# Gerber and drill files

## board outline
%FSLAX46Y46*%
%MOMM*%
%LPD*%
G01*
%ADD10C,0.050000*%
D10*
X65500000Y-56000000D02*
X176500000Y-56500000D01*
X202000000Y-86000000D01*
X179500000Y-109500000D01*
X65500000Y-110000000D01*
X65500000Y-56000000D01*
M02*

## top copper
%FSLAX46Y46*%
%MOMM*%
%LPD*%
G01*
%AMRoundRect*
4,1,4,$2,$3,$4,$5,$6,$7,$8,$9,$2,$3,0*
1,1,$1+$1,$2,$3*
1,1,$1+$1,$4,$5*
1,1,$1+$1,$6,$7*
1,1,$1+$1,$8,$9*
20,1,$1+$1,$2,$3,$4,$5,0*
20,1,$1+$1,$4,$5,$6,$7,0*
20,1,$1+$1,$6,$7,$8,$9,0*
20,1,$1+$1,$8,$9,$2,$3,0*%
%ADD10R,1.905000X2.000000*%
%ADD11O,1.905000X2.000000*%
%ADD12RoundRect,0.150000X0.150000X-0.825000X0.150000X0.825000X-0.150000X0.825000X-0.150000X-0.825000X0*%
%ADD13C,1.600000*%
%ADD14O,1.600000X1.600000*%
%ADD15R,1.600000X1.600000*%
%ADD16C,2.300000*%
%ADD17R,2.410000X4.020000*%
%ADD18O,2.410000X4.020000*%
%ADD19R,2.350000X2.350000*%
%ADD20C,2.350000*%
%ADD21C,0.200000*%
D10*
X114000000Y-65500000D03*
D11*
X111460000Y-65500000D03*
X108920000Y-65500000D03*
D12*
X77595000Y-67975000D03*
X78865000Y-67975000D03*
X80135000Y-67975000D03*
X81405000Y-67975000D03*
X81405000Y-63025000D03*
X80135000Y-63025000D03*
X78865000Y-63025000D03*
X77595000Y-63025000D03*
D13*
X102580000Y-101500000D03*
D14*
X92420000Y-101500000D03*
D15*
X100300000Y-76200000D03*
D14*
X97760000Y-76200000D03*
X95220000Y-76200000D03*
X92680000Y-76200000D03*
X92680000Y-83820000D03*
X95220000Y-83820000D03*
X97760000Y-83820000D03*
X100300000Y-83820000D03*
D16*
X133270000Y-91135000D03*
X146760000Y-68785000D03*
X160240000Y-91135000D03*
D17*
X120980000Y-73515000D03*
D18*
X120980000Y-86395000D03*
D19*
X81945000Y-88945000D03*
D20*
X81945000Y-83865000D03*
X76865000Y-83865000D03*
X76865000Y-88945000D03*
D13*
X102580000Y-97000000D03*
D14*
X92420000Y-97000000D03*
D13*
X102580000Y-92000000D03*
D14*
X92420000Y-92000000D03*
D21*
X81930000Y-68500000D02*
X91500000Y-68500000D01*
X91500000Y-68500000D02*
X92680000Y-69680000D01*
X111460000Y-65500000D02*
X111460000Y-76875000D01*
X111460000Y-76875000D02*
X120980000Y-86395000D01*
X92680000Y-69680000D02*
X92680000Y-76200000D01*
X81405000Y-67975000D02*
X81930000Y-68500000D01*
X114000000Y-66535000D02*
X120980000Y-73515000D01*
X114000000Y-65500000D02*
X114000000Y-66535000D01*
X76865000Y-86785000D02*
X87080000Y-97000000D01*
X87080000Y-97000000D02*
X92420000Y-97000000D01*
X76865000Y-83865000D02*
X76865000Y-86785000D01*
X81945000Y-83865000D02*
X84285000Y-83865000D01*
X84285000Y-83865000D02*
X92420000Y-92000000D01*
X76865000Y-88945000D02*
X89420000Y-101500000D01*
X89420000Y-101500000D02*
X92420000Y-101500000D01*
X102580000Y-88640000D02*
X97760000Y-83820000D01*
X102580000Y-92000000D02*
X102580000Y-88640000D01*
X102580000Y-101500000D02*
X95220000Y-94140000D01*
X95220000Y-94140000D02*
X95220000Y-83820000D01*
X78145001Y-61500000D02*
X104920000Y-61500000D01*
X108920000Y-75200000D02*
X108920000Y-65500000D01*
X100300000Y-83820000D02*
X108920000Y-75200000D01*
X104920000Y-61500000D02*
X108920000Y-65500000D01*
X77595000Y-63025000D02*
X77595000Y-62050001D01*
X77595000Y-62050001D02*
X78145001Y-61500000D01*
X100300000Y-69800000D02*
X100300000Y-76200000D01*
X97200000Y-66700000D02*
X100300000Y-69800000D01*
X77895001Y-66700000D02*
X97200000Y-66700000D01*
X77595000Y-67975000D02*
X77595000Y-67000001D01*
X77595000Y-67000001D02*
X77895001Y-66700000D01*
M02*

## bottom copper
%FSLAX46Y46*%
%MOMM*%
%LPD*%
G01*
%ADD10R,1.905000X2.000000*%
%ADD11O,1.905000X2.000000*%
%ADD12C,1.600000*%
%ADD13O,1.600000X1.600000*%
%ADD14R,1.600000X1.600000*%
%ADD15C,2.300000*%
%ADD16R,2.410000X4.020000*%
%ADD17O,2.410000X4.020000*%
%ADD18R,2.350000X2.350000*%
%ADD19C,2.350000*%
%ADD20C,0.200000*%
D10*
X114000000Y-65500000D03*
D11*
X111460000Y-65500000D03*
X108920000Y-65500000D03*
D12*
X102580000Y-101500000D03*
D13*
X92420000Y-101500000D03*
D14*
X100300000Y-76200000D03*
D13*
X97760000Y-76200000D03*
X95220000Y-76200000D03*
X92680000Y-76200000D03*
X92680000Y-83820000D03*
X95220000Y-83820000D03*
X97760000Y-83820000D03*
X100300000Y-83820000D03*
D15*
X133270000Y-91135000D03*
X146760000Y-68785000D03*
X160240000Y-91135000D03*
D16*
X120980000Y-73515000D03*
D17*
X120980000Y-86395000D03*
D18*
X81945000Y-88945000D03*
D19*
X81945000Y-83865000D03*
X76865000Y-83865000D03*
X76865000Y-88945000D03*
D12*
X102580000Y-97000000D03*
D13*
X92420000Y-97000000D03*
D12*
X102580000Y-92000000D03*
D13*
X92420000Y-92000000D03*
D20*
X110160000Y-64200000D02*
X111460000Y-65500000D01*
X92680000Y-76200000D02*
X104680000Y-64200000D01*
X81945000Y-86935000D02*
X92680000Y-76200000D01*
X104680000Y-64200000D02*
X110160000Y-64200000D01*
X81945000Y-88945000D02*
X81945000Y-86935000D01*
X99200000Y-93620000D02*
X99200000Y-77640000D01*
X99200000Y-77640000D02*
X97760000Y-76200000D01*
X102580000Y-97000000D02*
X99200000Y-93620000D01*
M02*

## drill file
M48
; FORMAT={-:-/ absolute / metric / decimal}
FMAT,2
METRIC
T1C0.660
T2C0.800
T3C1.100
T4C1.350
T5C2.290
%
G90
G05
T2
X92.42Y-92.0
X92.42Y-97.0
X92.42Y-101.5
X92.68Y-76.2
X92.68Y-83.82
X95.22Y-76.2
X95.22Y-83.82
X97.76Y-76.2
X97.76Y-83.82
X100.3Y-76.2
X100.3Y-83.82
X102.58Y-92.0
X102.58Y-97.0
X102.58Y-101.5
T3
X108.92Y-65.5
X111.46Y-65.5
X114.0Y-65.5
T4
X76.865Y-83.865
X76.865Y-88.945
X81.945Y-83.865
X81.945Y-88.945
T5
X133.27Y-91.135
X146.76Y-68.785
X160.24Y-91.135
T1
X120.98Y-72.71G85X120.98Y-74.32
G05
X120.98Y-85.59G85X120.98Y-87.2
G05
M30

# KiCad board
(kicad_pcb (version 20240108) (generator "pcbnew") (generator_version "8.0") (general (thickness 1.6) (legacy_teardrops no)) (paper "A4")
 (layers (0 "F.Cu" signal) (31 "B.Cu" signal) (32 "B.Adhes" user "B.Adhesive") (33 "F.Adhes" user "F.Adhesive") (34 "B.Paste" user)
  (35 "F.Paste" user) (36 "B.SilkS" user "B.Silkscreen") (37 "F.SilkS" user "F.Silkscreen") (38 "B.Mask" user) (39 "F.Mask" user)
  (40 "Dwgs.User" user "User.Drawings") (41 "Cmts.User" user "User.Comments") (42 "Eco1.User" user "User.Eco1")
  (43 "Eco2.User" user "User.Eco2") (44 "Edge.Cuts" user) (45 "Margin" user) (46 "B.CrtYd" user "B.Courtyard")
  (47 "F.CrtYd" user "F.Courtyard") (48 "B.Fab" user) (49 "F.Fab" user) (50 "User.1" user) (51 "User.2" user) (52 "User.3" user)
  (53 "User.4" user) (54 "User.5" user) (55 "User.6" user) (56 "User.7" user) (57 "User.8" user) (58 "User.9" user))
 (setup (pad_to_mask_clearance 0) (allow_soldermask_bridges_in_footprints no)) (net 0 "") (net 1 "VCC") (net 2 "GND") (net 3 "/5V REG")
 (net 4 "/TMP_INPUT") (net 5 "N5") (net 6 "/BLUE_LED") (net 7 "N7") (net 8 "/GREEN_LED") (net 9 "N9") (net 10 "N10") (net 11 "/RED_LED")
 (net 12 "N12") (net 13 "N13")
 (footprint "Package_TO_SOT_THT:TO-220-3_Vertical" (layer "F.Cu") (at 114 65.5 180)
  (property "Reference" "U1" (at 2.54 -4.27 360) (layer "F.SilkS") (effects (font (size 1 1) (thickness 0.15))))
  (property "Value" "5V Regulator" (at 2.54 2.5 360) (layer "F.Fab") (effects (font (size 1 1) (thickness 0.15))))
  (pad "1" thru_hole rect (at 0 0 180) (size 1.905 2) (drill 1.1) (layers "*.Cu" "*.Mask") (remove_unused_layers no) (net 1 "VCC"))
  (pad "2" thru_hole oval (at 2.54 0 180) (size 1.905 2) (drill 1.1) (layers "*.Cu" "*.Mask") (remove_unused_layers no) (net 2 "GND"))
  (pad "3" thru_hole oval (at 5.08 0 180) (size 1.905 2) (drill 1.1) (layers "*.Cu" "*.Mask") (remove_unused_layers no) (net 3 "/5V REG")))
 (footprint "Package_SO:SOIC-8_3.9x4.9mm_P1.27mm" (layer "F.Cu") (at 79.5 65.5 90)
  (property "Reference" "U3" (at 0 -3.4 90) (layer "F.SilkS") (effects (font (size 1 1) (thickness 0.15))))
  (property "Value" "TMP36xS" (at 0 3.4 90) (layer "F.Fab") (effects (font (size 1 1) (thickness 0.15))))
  (pad "1" smd roundrect (at -2.475 -1.905 90) (size 1.95 0.6) (layers "F.Cu" "F.Paste" "F.Mask") (roundrect_rratio 0.25)
   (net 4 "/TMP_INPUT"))
  (pad "2" smd roundrect (at -2.475 -0.635 90) (size 1.95 0.6) (layers "F.Cu" "F.Paste" "F.Mask") (roundrect_rratio 0.25))
  (pad "3" smd roundrect (at -2.475 0.635 90) (size 1.95 0.6) (layers "F.Cu" "F.Paste" "F.Mask") (roundrect_rratio 0.25))
  (pad "4" smd roundrect (at -2.475 1.905 90) (size 1.95 0.6) (layers "F.Cu" "F.Paste" "F.Mask") (roundrect_rratio 0.25) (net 2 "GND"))
  (pad "5" smd roundrect (at 2.475 1.905 90) (size 1.95 0.6) (layers "F.Cu" "F.Paste" "F.Mask") (roundrect_rratio 0.25) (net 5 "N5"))
  (pad "6" smd roundrect (at 2.475 0.635 90) (size 1.95 0.6) (layers "F.Cu" "F.Paste" "F.Mask") (roundrect_rratio 0.25))
  (pad "7" smd roundrect (at 2.475 -0.635 90) (size 1.95 0.6) (layers "F.Cu" "F.Paste" "F.Mask") (roundrect_rratio 0.25))
  (pad "8" smd roundrect (at 2.475 -1.905 90) (size 1.95 0.6) (layers "F.Cu" "F.Paste" "F.Mask") (roundrect_rratio 0.25) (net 3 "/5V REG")))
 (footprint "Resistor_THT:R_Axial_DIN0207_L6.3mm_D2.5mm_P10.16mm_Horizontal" (layer "F.Cu") (at 102.58 101.5 180)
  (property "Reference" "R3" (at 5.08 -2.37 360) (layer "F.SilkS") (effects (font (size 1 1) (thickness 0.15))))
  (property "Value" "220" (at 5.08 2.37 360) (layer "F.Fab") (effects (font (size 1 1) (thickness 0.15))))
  (pad "1" thru_hole circle (at 0 0 180) (size 1.6 1.6) (drill 0.8) (layers "*.Cu" "*.Mask") (remove_unused_layers no) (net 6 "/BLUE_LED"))
  (pad "2" thru_hole oval (at 10.16 0 180) (size 1.6 1.6) (drill 0.8) (layers "*.Cu" "*.Mask") (remove_unused_layers no) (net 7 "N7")))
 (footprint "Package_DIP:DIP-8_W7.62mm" (layer "F.Cu") (at 100.3 76.2 -90)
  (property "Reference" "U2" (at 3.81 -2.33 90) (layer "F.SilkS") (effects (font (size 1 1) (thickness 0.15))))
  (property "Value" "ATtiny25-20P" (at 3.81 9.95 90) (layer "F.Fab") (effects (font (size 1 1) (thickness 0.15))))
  (pad "1" thru_hole rect (at 0 0 270) (size 1.6 1.6) (drill 0.8) (layers "*.Cu" "*.Mask") (remove_unused_layers no) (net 4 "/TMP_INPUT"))
  (pad "2" thru_hole oval (at 0 2.54 270) (size 1.6 1.6) (drill 0.8) (layers "*.Cu" "*.Mask") (remove_unused_layers no) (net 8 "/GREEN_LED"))
  (pad "3" thru_hole oval (at 0 5.08 270) (size 1.6 1.6) (drill 0.8) (layers "*.Cu" "*.Mask") (remove_unused_layers no) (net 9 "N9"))
  (pad "4" thru_hole oval (at 0 7.62 270) (size 1.6 1.6) (drill 0.8) (layers "*.Cu" "*.Mask") (remove_unused_layers no) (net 2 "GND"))
  (pad "5" thru_hole oval (at 7.62 7.62 270) (size 1.6 1.6) (drill 0.8) (layers "*.Cu" "*.Mask") (remove_unused_layers no) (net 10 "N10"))
  (pad "6" thru_hole oval (at 7.62 5.08 270) (size 1.6 1.6) (drill 0.8) (layers "*.Cu" "*.Mask") (remove_unused_layers no)
   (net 6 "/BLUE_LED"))
  (pad "7" thru_hole oval (at 7.62 2.54 270) (size 1.6 1.6) (drill 0.8) (layers "*.Cu" "*.Mask") (remove_unused_layers no)
   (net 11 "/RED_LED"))
  (pad "8" thru_hole oval (at 7.62 0 270) (size 1.6 1.6) (drill 0.8) (layers "*.Cu" "*.Mask") (remove_unused_layers no) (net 3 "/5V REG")))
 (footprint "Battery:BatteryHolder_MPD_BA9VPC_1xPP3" (layer "F.Cu") (at 120.98 73.515)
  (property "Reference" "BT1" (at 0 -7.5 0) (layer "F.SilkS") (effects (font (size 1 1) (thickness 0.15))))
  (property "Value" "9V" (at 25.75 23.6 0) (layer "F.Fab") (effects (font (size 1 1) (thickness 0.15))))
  (pad "" np_thru_hole circle (at 12.29 17.62) (size 2.3 2.3) (drill 2.29) (layers "*.Cu" "*.Mask"))
  (pad "" np_thru_hole circle (at 25.78 -4.73) (size 2.3 2.3) (drill 2.29) (layers "*.Cu" "*.Mask"))
  (pad "" np_thru_hole circle (at 39.26 17.62) (size 2.3 2.3) (drill 2.29) (layers "*.Cu" "*.Mask"))
  (pad "1" thru_hole rect (at 0 0) (size 2.41 4.02) (drill oval 0.66 2.27) (layers "*.Cu" "*.Mask") (remove_unused_layers no) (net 1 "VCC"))
  (pad "2" thru_hole oval (at 0 12.88) (size 2.41 4.02) (drill oval 0.66 2.27) (layers "*.Cu" "*.Mask") (remove_unused_layers no)
   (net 2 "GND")))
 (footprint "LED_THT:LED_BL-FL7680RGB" (layer "F.Cu") (at 81.945 88.945 180)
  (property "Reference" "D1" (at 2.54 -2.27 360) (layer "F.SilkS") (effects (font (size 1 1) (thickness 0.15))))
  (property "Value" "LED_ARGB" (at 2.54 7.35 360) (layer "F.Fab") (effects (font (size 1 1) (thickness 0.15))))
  (pad "1" thru_hole rect (at 0 0 180) (size 2.35 2.35) (drill 1.35) (layers "*.Cu" "*.Mask") (remove_unused_layers no) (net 2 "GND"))
  (pad "2" thru_hole circle (at 0 5.08 180) (size 2.35 2.35) (drill 1.35) (layers "*.Cu" "*.Mask") (remove_unused_layers no) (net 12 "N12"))
  (pad "3" thru_hole circle (at 5.08 5.08 180) (size 2.35 2.35) (drill 1.35) (layers "*.Cu" "*.Mask") (remove_unused_layers no)
   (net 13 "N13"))
  (pad "4" thru_hole circle (at 5.08 0 180) (size 2.35 2.35) (drill 1.35) (layers "*.Cu" "*.Mask") (remove_unused_layers no) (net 7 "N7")))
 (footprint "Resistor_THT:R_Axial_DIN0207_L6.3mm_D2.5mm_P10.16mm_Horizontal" (layer "F.Cu") (at 102.58 97 180)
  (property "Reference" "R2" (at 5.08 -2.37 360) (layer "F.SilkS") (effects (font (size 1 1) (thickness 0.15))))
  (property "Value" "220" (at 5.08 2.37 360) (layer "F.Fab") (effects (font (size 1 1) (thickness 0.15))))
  (pad "1" thru_hole circle (at 0 0 180) (size 1.6 1.6) (drill 0.8) (layers "*.Cu" "*.Mask") (remove_unused_layers no) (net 8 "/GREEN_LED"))
  (pad "2" thru_hole oval (at 10.16 0 180) (size 1.6 1.6) (drill 0.8) (layers "*.Cu" "*.Mask") (remove_unused_layers no) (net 13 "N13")))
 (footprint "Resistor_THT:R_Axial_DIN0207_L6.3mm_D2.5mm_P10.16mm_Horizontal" (layer "F.Cu") (at 102.58 92 180)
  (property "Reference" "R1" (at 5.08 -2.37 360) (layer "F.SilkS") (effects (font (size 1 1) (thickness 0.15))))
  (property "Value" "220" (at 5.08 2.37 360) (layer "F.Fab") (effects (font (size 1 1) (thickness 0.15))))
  (pad "1" thru_hole circle (at 0 0 180) (size 1.6 1.6) (drill 0.8) (layers "*.Cu" "*.Mask") (remove_unused_layers no) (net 11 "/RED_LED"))
  (pad "2" thru_hole oval (at 10.16 0 180) (size 1.6 1.6) (drill 0.8) (layers "*.Cu" "*.Mask") (remove_unused_layers no) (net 12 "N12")))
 (gr_poly
  (pts (xy 65.5 56) (xy 176.5 56.5) (xy 202 86) (xy 179.5 109.5) (xy 65.5 110)) (stroke (width 0.05) (type solid)) (fill none)
  (layer "Edge.Cuts"))
 (segment (start 81.93 68.5) (end 91.5 68.5) (width 0.2) (layer "F.Cu") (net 2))
 (segment (start 91.5 68.5) (end 92.68 69.68) (width 0.2) (layer "F.Cu") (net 2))
 (segment (start 111.46 65.5) (end 111.46 76.875) (width 0.2) (layer "F.Cu") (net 2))
 (segment (start 111.46 76.875) (end 120.98 86.395) (width 0.2) (layer "F.Cu") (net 2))
 (segment (start 92.68 69.68) (end 92.68 76.2) (width 0.2) (layer "F.Cu") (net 2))
 (segment (start 81.405 67.975) (end 81.93 68.5) (width 0.2) (layer "F.Cu") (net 2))
 (segment (start 110.16 64.2) (end 111.46 65.5) (width 0.2) (layer "B.Cu") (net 2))
 (segment (start 92.68 76.2) (end 104.68 64.2) (width 0.2) (layer "B.Cu") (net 2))
 (segment (start 81.945 86.935) (end 92.68 76.2) (width 0.2) (layer "B.Cu") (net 2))
 (segment (start 104.68 64.2) (end 110.16 64.2) (width 0.2) (layer "B.Cu") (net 2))
 (segment (start 81.945 88.945) (end 81.945 86.935) (width 0.2) (layer "B.Cu") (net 2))
 (segment (start 114 66.535) (end 120.98 73.515) (width 0.2) (layer "F.Cu") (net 1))
 (segment (start 114 65.5) (end 114 66.535) (width 0.2) (layer "F.Cu") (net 1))
 (segment (start 76.865 86.785) (end 87.08 97) (width 0.2) (layer "F.Cu") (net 13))
 (segment (start 87.08 97) (end 92.42 97) (width 0.2) (layer "F.Cu") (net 13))
 (segment (start 76.865 83.865) (end 76.865 86.785) (width 0.2) (layer "F.Cu") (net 13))
 (segment (start 81.945 83.865) (end 84.285 83.865) (width 0.2) (layer "F.Cu") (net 12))
 (segment (start 84.285 83.865) (end 92.42 92) (width 0.2) (layer "F.Cu") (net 12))
 (segment (start 76.865 88.945) (end 89.42 101.5) (width 0.2) (layer "F.Cu") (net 7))
 (segment (start 89.42 101.5) (end 92.42 101.5) (width 0.2) (layer "F.Cu") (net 7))
 (segment (start 102.58 88.64) (end 97.76 83.82) (width 0.2) (layer "F.Cu") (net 11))
 (segment (start 102.58 92) (end 102.58 88.64) (width 0.2) (layer "F.Cu") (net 11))
 (segment (start 99.2 93.62) (end 99.2 77.64) (width 0.2) (layer "B.Cu") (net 8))
 (segment (start 99.2 77.64) (end 97.76 76.2) (width 0.2) (layer "B.Cu") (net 8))
 (segment (start 102.58 97) (end 99.2 93.62) (width 0.2) (layer "B.Cu") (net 8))
 (segment (start 102.58 101.5) (end 95.22 94.14) (width 0.2) (layer "F.Cu") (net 6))
 (segment (start 95.22 94.14) (end 95.22 83.82) (width 0.2) (layer "F.Cu") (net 6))
 (segment (start 78.145001 61.5) (end 104.92 61.5) (width 0.2) (layer "F.Cu") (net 3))
 (segment (start 108.92 75.2) (end 108.92 65.5) (width 0.2) (layer "F.Cu") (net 3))
 (segment (start 100.3 83.82) (end 108.92 75.2) (width 0.2) (layer "F.Cu") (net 3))
 (segment (start 104.92 61.5) (end 108.92 65.5) (width 0.2) (layer "F.Cu") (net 3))
 (segment (start 77.595 63.025) (end 77.595 62.050001) (width 0.2) (layer "F.Cu") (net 3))
 (segment (start 77.595 62.050001) (end 78.145001 61.5) (width 0.2) (layer "F.Cu") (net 3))
 (segment (start 100.3 69.8) (end 100.3 76.2) (width 0.2) (layer "F.Cu") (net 4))
 (segment (start 97.2 66.7) (end 100.3 69.8) (width 0.2) (layer "F.Cu") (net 4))
 (segment (start 77.895001 66.7) (end 97.2 66.7) (width 0.2) (layer "F.Cu") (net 4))
 (segment (start 77.595 67.975) (end 77.595 67.000001) (width 0.2) (layer "F.Cu") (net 4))
 (segment (start 77.595 67.000001) (end 77.895001 66.7) (width 0.2) (layer "F.Cu") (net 4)))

